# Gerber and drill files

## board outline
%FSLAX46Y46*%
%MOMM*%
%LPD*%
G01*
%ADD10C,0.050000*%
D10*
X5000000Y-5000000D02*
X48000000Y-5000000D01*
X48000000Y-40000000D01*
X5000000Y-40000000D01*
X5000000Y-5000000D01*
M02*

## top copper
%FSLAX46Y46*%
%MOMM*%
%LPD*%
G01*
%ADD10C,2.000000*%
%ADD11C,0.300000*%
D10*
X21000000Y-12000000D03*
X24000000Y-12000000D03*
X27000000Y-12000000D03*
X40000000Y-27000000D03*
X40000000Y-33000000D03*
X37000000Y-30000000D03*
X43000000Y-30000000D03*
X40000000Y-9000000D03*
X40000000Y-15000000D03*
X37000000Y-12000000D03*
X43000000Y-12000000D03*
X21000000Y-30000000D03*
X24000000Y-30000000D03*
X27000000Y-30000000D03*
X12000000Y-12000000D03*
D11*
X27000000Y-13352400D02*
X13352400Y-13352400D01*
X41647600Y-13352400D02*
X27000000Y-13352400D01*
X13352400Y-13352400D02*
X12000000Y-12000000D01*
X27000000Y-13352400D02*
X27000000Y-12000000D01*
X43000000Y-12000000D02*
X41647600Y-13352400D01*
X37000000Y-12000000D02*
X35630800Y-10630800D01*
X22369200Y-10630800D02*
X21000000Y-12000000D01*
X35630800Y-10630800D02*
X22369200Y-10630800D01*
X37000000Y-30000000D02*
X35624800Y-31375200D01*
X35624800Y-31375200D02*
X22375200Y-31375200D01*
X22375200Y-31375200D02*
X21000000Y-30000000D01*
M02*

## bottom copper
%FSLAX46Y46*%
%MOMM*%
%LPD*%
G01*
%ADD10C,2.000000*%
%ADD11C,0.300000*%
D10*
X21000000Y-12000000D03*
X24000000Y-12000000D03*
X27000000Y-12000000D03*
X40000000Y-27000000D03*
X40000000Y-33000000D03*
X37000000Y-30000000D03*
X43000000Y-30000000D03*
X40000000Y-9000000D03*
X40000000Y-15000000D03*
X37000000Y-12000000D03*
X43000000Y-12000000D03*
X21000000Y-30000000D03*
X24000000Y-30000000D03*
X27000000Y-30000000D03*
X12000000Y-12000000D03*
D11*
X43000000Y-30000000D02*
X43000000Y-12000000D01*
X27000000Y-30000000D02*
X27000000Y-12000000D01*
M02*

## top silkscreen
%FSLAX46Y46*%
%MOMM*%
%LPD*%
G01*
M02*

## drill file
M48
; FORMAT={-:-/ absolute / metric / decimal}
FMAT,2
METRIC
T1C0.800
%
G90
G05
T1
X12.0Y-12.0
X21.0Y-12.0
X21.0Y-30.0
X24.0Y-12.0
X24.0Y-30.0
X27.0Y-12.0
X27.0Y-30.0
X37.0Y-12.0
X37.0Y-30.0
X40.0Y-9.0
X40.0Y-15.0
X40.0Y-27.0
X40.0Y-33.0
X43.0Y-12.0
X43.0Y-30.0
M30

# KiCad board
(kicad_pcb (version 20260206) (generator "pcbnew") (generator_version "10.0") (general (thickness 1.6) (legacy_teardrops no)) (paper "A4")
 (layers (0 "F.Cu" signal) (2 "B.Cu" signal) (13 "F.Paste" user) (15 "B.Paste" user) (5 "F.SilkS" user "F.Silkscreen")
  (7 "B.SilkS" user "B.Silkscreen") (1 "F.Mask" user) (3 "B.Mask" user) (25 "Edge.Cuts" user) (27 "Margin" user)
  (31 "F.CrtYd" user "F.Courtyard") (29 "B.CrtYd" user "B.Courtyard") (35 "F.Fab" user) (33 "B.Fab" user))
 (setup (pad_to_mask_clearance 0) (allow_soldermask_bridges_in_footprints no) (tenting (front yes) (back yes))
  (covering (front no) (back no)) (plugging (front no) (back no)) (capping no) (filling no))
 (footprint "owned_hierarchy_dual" (layer "F.Cu") (at 24 12)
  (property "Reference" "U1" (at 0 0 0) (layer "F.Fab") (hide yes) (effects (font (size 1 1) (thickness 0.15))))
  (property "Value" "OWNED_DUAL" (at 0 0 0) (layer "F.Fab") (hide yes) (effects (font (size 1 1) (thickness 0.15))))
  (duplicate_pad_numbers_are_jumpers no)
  (pad "1" thru_hole circle (at -3 0) (size 2 2) (drill 0.8) (layers "*.Cu" "*.Mask") (remove_unused_layers no) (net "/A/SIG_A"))
  (pad "2" thru_hole circle (at 0 0) (size 2 2) (drill 0.8) (layers "*.Cu" "*.Mask") (remove_unused_layers no) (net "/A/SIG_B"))
  (pad "3" thru_hole circle (at 3 0) (size 2 2) (drill 0.8) (layers "*.Cu" "*.Mask") (remove_unused_layers no) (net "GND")))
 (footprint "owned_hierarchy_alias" (layer "F.Cu") (at 40 30)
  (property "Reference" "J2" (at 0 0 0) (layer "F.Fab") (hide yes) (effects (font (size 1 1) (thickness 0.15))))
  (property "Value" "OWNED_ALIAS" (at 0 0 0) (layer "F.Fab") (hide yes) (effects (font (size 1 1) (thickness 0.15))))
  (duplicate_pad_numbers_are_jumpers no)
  (pad "MP" thru_hole circle (at 0 -3) (size 2 2) (drill 0.8) (layers "*.Cu" "*.Mask") (remove_unused_layers no))
  (pad "MP" thru_hole circle (at 0 3) (size 2 2) (drill 0.8) (layers "*.Cu" "*.Mask") (remove_unused_layers no))
  (pad "R" thru_hole circle (at -3 0) (size 2 2) (drill 0.8) (layers "*.Cu" "*.Mask") (remove_unused_layers no) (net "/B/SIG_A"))
  (pad "T" thru_hole circle (at 3 0) (size 2 2) (drill 0.8) (layers "*.Cu" "*.Mask") (remove_unused_layers no) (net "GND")))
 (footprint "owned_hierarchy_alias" (layer "F.Cu") (at 40 12)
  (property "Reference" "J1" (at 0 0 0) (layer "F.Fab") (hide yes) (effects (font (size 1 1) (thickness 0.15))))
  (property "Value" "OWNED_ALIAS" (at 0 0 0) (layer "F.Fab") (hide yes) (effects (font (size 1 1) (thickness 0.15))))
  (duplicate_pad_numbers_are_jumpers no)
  (pad "MP" thru_hole circle (at 0 -3) (size 2 2) (drill 0.8) (layers "*.Cu" "*.Mask") (remove_unused_layers no))
  (pad "MP" thru_hole circle (at 0 3) (size 2 2) (drill 0.8) (layers "*.Cu" "*.Mask") (remove_unused_layers no))
  (pad "R" thru_hole circle (at -3 0) (size 2 2) (drill 0.8) (layers "*.Cu" "*.Mask") (remove_unused_layers no) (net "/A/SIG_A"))
  (pad "T" thru_hole circle (at 3 0) (size 2 2) (drill 0.8) (layers "*.Cu" "*.Mask") (remove_unused_layers no) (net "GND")))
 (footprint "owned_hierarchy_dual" (layer "F.Cu") (at 24 30)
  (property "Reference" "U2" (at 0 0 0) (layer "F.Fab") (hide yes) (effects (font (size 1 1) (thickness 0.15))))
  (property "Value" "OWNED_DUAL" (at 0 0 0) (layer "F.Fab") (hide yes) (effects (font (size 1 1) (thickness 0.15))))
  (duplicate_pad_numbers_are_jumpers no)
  (pad "1" thru_hole circle (at -3 0) (size 2 2) (drill 0.8) (layers "*.Cu" "*.Mask") (remove_unused_layers no) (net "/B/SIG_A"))
  (pad "2" thru_hole circle (at 0 0) (size 2 2) (drill 0.8) (layers "*.Cu" "*.Mask") (remove_unused_layers no) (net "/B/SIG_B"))
  (pad "3" thru_hole circle (at 3 0) (size 2 2) (drill 0.8) (layers "*.Cu" "*.Mask") (remove_unused_layers no) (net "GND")))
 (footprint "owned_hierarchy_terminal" (layer "F.Cu") (at 12 12)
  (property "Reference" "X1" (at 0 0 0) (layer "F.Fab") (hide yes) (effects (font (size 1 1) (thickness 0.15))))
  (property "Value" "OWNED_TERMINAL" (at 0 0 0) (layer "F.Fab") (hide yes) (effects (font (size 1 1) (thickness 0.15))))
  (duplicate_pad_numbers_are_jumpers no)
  (pad "1" thru_hole circle (at 0 0) (size 2 2) (drill 0.8) (layers "*.Cu" "*.Mask") (remove_unused_layers no) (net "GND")))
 (gr_rect (start 5 5) (end 48 40) (stroke (width 0.05) (type default)) (fill no) (layer "Edge.Cuts"))
 (segment (start 27 13.3524) (end 13.3524 13.3524) (width 0.3) (layer "F.Cu") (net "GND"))
 (segment (start 41.6476 13.3524) (end 27 13.3524) (width 0.3) (layer "F.Cu") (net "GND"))
 (segment (start 13.3524 13.3524) (end 12 12) (width 0.3) (layer "F.Cu") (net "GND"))
 (segment (start 27 13.3524) (end 27 12) (width 0.3) (layer "F.Cu") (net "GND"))
 (segment (start 43 12) (end 41.6476 13.3524) (width 0.3) (layer "F.Cu") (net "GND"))
 (segment (start 43 30) (end 43 12) (width 0.3) (layer "B.Cu") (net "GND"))
 (segment (start 27 30) (end 27 12) (width 0.3) (layer "B.Cu") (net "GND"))
 (segment (start 37 12) (end 35.6308 10.6308) (width 0.3) (layer "F.Cu") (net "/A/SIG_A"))
 (segment (start 22.3692 10.6308) (end 21 12) (width 0.3) (layer "F.Cu") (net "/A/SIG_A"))
 (segment (start 35.6308 10.6308) (end 22.3692 10.6308) (width 0.3) (layer "F.Cu") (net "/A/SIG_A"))
 (segment (start 37 30) (end 35.6248 31.3752) (width 0.3) (layer "F.Cu") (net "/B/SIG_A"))
 (segment (start 35.6248 31.3752) (end 22.3752 31.3752) (width 0.3) (layer "F.Cu") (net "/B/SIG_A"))
 (segment (start 22.3752 31.3752) (end 21 30) (width 0.3) (layer "F.Cu") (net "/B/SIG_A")))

